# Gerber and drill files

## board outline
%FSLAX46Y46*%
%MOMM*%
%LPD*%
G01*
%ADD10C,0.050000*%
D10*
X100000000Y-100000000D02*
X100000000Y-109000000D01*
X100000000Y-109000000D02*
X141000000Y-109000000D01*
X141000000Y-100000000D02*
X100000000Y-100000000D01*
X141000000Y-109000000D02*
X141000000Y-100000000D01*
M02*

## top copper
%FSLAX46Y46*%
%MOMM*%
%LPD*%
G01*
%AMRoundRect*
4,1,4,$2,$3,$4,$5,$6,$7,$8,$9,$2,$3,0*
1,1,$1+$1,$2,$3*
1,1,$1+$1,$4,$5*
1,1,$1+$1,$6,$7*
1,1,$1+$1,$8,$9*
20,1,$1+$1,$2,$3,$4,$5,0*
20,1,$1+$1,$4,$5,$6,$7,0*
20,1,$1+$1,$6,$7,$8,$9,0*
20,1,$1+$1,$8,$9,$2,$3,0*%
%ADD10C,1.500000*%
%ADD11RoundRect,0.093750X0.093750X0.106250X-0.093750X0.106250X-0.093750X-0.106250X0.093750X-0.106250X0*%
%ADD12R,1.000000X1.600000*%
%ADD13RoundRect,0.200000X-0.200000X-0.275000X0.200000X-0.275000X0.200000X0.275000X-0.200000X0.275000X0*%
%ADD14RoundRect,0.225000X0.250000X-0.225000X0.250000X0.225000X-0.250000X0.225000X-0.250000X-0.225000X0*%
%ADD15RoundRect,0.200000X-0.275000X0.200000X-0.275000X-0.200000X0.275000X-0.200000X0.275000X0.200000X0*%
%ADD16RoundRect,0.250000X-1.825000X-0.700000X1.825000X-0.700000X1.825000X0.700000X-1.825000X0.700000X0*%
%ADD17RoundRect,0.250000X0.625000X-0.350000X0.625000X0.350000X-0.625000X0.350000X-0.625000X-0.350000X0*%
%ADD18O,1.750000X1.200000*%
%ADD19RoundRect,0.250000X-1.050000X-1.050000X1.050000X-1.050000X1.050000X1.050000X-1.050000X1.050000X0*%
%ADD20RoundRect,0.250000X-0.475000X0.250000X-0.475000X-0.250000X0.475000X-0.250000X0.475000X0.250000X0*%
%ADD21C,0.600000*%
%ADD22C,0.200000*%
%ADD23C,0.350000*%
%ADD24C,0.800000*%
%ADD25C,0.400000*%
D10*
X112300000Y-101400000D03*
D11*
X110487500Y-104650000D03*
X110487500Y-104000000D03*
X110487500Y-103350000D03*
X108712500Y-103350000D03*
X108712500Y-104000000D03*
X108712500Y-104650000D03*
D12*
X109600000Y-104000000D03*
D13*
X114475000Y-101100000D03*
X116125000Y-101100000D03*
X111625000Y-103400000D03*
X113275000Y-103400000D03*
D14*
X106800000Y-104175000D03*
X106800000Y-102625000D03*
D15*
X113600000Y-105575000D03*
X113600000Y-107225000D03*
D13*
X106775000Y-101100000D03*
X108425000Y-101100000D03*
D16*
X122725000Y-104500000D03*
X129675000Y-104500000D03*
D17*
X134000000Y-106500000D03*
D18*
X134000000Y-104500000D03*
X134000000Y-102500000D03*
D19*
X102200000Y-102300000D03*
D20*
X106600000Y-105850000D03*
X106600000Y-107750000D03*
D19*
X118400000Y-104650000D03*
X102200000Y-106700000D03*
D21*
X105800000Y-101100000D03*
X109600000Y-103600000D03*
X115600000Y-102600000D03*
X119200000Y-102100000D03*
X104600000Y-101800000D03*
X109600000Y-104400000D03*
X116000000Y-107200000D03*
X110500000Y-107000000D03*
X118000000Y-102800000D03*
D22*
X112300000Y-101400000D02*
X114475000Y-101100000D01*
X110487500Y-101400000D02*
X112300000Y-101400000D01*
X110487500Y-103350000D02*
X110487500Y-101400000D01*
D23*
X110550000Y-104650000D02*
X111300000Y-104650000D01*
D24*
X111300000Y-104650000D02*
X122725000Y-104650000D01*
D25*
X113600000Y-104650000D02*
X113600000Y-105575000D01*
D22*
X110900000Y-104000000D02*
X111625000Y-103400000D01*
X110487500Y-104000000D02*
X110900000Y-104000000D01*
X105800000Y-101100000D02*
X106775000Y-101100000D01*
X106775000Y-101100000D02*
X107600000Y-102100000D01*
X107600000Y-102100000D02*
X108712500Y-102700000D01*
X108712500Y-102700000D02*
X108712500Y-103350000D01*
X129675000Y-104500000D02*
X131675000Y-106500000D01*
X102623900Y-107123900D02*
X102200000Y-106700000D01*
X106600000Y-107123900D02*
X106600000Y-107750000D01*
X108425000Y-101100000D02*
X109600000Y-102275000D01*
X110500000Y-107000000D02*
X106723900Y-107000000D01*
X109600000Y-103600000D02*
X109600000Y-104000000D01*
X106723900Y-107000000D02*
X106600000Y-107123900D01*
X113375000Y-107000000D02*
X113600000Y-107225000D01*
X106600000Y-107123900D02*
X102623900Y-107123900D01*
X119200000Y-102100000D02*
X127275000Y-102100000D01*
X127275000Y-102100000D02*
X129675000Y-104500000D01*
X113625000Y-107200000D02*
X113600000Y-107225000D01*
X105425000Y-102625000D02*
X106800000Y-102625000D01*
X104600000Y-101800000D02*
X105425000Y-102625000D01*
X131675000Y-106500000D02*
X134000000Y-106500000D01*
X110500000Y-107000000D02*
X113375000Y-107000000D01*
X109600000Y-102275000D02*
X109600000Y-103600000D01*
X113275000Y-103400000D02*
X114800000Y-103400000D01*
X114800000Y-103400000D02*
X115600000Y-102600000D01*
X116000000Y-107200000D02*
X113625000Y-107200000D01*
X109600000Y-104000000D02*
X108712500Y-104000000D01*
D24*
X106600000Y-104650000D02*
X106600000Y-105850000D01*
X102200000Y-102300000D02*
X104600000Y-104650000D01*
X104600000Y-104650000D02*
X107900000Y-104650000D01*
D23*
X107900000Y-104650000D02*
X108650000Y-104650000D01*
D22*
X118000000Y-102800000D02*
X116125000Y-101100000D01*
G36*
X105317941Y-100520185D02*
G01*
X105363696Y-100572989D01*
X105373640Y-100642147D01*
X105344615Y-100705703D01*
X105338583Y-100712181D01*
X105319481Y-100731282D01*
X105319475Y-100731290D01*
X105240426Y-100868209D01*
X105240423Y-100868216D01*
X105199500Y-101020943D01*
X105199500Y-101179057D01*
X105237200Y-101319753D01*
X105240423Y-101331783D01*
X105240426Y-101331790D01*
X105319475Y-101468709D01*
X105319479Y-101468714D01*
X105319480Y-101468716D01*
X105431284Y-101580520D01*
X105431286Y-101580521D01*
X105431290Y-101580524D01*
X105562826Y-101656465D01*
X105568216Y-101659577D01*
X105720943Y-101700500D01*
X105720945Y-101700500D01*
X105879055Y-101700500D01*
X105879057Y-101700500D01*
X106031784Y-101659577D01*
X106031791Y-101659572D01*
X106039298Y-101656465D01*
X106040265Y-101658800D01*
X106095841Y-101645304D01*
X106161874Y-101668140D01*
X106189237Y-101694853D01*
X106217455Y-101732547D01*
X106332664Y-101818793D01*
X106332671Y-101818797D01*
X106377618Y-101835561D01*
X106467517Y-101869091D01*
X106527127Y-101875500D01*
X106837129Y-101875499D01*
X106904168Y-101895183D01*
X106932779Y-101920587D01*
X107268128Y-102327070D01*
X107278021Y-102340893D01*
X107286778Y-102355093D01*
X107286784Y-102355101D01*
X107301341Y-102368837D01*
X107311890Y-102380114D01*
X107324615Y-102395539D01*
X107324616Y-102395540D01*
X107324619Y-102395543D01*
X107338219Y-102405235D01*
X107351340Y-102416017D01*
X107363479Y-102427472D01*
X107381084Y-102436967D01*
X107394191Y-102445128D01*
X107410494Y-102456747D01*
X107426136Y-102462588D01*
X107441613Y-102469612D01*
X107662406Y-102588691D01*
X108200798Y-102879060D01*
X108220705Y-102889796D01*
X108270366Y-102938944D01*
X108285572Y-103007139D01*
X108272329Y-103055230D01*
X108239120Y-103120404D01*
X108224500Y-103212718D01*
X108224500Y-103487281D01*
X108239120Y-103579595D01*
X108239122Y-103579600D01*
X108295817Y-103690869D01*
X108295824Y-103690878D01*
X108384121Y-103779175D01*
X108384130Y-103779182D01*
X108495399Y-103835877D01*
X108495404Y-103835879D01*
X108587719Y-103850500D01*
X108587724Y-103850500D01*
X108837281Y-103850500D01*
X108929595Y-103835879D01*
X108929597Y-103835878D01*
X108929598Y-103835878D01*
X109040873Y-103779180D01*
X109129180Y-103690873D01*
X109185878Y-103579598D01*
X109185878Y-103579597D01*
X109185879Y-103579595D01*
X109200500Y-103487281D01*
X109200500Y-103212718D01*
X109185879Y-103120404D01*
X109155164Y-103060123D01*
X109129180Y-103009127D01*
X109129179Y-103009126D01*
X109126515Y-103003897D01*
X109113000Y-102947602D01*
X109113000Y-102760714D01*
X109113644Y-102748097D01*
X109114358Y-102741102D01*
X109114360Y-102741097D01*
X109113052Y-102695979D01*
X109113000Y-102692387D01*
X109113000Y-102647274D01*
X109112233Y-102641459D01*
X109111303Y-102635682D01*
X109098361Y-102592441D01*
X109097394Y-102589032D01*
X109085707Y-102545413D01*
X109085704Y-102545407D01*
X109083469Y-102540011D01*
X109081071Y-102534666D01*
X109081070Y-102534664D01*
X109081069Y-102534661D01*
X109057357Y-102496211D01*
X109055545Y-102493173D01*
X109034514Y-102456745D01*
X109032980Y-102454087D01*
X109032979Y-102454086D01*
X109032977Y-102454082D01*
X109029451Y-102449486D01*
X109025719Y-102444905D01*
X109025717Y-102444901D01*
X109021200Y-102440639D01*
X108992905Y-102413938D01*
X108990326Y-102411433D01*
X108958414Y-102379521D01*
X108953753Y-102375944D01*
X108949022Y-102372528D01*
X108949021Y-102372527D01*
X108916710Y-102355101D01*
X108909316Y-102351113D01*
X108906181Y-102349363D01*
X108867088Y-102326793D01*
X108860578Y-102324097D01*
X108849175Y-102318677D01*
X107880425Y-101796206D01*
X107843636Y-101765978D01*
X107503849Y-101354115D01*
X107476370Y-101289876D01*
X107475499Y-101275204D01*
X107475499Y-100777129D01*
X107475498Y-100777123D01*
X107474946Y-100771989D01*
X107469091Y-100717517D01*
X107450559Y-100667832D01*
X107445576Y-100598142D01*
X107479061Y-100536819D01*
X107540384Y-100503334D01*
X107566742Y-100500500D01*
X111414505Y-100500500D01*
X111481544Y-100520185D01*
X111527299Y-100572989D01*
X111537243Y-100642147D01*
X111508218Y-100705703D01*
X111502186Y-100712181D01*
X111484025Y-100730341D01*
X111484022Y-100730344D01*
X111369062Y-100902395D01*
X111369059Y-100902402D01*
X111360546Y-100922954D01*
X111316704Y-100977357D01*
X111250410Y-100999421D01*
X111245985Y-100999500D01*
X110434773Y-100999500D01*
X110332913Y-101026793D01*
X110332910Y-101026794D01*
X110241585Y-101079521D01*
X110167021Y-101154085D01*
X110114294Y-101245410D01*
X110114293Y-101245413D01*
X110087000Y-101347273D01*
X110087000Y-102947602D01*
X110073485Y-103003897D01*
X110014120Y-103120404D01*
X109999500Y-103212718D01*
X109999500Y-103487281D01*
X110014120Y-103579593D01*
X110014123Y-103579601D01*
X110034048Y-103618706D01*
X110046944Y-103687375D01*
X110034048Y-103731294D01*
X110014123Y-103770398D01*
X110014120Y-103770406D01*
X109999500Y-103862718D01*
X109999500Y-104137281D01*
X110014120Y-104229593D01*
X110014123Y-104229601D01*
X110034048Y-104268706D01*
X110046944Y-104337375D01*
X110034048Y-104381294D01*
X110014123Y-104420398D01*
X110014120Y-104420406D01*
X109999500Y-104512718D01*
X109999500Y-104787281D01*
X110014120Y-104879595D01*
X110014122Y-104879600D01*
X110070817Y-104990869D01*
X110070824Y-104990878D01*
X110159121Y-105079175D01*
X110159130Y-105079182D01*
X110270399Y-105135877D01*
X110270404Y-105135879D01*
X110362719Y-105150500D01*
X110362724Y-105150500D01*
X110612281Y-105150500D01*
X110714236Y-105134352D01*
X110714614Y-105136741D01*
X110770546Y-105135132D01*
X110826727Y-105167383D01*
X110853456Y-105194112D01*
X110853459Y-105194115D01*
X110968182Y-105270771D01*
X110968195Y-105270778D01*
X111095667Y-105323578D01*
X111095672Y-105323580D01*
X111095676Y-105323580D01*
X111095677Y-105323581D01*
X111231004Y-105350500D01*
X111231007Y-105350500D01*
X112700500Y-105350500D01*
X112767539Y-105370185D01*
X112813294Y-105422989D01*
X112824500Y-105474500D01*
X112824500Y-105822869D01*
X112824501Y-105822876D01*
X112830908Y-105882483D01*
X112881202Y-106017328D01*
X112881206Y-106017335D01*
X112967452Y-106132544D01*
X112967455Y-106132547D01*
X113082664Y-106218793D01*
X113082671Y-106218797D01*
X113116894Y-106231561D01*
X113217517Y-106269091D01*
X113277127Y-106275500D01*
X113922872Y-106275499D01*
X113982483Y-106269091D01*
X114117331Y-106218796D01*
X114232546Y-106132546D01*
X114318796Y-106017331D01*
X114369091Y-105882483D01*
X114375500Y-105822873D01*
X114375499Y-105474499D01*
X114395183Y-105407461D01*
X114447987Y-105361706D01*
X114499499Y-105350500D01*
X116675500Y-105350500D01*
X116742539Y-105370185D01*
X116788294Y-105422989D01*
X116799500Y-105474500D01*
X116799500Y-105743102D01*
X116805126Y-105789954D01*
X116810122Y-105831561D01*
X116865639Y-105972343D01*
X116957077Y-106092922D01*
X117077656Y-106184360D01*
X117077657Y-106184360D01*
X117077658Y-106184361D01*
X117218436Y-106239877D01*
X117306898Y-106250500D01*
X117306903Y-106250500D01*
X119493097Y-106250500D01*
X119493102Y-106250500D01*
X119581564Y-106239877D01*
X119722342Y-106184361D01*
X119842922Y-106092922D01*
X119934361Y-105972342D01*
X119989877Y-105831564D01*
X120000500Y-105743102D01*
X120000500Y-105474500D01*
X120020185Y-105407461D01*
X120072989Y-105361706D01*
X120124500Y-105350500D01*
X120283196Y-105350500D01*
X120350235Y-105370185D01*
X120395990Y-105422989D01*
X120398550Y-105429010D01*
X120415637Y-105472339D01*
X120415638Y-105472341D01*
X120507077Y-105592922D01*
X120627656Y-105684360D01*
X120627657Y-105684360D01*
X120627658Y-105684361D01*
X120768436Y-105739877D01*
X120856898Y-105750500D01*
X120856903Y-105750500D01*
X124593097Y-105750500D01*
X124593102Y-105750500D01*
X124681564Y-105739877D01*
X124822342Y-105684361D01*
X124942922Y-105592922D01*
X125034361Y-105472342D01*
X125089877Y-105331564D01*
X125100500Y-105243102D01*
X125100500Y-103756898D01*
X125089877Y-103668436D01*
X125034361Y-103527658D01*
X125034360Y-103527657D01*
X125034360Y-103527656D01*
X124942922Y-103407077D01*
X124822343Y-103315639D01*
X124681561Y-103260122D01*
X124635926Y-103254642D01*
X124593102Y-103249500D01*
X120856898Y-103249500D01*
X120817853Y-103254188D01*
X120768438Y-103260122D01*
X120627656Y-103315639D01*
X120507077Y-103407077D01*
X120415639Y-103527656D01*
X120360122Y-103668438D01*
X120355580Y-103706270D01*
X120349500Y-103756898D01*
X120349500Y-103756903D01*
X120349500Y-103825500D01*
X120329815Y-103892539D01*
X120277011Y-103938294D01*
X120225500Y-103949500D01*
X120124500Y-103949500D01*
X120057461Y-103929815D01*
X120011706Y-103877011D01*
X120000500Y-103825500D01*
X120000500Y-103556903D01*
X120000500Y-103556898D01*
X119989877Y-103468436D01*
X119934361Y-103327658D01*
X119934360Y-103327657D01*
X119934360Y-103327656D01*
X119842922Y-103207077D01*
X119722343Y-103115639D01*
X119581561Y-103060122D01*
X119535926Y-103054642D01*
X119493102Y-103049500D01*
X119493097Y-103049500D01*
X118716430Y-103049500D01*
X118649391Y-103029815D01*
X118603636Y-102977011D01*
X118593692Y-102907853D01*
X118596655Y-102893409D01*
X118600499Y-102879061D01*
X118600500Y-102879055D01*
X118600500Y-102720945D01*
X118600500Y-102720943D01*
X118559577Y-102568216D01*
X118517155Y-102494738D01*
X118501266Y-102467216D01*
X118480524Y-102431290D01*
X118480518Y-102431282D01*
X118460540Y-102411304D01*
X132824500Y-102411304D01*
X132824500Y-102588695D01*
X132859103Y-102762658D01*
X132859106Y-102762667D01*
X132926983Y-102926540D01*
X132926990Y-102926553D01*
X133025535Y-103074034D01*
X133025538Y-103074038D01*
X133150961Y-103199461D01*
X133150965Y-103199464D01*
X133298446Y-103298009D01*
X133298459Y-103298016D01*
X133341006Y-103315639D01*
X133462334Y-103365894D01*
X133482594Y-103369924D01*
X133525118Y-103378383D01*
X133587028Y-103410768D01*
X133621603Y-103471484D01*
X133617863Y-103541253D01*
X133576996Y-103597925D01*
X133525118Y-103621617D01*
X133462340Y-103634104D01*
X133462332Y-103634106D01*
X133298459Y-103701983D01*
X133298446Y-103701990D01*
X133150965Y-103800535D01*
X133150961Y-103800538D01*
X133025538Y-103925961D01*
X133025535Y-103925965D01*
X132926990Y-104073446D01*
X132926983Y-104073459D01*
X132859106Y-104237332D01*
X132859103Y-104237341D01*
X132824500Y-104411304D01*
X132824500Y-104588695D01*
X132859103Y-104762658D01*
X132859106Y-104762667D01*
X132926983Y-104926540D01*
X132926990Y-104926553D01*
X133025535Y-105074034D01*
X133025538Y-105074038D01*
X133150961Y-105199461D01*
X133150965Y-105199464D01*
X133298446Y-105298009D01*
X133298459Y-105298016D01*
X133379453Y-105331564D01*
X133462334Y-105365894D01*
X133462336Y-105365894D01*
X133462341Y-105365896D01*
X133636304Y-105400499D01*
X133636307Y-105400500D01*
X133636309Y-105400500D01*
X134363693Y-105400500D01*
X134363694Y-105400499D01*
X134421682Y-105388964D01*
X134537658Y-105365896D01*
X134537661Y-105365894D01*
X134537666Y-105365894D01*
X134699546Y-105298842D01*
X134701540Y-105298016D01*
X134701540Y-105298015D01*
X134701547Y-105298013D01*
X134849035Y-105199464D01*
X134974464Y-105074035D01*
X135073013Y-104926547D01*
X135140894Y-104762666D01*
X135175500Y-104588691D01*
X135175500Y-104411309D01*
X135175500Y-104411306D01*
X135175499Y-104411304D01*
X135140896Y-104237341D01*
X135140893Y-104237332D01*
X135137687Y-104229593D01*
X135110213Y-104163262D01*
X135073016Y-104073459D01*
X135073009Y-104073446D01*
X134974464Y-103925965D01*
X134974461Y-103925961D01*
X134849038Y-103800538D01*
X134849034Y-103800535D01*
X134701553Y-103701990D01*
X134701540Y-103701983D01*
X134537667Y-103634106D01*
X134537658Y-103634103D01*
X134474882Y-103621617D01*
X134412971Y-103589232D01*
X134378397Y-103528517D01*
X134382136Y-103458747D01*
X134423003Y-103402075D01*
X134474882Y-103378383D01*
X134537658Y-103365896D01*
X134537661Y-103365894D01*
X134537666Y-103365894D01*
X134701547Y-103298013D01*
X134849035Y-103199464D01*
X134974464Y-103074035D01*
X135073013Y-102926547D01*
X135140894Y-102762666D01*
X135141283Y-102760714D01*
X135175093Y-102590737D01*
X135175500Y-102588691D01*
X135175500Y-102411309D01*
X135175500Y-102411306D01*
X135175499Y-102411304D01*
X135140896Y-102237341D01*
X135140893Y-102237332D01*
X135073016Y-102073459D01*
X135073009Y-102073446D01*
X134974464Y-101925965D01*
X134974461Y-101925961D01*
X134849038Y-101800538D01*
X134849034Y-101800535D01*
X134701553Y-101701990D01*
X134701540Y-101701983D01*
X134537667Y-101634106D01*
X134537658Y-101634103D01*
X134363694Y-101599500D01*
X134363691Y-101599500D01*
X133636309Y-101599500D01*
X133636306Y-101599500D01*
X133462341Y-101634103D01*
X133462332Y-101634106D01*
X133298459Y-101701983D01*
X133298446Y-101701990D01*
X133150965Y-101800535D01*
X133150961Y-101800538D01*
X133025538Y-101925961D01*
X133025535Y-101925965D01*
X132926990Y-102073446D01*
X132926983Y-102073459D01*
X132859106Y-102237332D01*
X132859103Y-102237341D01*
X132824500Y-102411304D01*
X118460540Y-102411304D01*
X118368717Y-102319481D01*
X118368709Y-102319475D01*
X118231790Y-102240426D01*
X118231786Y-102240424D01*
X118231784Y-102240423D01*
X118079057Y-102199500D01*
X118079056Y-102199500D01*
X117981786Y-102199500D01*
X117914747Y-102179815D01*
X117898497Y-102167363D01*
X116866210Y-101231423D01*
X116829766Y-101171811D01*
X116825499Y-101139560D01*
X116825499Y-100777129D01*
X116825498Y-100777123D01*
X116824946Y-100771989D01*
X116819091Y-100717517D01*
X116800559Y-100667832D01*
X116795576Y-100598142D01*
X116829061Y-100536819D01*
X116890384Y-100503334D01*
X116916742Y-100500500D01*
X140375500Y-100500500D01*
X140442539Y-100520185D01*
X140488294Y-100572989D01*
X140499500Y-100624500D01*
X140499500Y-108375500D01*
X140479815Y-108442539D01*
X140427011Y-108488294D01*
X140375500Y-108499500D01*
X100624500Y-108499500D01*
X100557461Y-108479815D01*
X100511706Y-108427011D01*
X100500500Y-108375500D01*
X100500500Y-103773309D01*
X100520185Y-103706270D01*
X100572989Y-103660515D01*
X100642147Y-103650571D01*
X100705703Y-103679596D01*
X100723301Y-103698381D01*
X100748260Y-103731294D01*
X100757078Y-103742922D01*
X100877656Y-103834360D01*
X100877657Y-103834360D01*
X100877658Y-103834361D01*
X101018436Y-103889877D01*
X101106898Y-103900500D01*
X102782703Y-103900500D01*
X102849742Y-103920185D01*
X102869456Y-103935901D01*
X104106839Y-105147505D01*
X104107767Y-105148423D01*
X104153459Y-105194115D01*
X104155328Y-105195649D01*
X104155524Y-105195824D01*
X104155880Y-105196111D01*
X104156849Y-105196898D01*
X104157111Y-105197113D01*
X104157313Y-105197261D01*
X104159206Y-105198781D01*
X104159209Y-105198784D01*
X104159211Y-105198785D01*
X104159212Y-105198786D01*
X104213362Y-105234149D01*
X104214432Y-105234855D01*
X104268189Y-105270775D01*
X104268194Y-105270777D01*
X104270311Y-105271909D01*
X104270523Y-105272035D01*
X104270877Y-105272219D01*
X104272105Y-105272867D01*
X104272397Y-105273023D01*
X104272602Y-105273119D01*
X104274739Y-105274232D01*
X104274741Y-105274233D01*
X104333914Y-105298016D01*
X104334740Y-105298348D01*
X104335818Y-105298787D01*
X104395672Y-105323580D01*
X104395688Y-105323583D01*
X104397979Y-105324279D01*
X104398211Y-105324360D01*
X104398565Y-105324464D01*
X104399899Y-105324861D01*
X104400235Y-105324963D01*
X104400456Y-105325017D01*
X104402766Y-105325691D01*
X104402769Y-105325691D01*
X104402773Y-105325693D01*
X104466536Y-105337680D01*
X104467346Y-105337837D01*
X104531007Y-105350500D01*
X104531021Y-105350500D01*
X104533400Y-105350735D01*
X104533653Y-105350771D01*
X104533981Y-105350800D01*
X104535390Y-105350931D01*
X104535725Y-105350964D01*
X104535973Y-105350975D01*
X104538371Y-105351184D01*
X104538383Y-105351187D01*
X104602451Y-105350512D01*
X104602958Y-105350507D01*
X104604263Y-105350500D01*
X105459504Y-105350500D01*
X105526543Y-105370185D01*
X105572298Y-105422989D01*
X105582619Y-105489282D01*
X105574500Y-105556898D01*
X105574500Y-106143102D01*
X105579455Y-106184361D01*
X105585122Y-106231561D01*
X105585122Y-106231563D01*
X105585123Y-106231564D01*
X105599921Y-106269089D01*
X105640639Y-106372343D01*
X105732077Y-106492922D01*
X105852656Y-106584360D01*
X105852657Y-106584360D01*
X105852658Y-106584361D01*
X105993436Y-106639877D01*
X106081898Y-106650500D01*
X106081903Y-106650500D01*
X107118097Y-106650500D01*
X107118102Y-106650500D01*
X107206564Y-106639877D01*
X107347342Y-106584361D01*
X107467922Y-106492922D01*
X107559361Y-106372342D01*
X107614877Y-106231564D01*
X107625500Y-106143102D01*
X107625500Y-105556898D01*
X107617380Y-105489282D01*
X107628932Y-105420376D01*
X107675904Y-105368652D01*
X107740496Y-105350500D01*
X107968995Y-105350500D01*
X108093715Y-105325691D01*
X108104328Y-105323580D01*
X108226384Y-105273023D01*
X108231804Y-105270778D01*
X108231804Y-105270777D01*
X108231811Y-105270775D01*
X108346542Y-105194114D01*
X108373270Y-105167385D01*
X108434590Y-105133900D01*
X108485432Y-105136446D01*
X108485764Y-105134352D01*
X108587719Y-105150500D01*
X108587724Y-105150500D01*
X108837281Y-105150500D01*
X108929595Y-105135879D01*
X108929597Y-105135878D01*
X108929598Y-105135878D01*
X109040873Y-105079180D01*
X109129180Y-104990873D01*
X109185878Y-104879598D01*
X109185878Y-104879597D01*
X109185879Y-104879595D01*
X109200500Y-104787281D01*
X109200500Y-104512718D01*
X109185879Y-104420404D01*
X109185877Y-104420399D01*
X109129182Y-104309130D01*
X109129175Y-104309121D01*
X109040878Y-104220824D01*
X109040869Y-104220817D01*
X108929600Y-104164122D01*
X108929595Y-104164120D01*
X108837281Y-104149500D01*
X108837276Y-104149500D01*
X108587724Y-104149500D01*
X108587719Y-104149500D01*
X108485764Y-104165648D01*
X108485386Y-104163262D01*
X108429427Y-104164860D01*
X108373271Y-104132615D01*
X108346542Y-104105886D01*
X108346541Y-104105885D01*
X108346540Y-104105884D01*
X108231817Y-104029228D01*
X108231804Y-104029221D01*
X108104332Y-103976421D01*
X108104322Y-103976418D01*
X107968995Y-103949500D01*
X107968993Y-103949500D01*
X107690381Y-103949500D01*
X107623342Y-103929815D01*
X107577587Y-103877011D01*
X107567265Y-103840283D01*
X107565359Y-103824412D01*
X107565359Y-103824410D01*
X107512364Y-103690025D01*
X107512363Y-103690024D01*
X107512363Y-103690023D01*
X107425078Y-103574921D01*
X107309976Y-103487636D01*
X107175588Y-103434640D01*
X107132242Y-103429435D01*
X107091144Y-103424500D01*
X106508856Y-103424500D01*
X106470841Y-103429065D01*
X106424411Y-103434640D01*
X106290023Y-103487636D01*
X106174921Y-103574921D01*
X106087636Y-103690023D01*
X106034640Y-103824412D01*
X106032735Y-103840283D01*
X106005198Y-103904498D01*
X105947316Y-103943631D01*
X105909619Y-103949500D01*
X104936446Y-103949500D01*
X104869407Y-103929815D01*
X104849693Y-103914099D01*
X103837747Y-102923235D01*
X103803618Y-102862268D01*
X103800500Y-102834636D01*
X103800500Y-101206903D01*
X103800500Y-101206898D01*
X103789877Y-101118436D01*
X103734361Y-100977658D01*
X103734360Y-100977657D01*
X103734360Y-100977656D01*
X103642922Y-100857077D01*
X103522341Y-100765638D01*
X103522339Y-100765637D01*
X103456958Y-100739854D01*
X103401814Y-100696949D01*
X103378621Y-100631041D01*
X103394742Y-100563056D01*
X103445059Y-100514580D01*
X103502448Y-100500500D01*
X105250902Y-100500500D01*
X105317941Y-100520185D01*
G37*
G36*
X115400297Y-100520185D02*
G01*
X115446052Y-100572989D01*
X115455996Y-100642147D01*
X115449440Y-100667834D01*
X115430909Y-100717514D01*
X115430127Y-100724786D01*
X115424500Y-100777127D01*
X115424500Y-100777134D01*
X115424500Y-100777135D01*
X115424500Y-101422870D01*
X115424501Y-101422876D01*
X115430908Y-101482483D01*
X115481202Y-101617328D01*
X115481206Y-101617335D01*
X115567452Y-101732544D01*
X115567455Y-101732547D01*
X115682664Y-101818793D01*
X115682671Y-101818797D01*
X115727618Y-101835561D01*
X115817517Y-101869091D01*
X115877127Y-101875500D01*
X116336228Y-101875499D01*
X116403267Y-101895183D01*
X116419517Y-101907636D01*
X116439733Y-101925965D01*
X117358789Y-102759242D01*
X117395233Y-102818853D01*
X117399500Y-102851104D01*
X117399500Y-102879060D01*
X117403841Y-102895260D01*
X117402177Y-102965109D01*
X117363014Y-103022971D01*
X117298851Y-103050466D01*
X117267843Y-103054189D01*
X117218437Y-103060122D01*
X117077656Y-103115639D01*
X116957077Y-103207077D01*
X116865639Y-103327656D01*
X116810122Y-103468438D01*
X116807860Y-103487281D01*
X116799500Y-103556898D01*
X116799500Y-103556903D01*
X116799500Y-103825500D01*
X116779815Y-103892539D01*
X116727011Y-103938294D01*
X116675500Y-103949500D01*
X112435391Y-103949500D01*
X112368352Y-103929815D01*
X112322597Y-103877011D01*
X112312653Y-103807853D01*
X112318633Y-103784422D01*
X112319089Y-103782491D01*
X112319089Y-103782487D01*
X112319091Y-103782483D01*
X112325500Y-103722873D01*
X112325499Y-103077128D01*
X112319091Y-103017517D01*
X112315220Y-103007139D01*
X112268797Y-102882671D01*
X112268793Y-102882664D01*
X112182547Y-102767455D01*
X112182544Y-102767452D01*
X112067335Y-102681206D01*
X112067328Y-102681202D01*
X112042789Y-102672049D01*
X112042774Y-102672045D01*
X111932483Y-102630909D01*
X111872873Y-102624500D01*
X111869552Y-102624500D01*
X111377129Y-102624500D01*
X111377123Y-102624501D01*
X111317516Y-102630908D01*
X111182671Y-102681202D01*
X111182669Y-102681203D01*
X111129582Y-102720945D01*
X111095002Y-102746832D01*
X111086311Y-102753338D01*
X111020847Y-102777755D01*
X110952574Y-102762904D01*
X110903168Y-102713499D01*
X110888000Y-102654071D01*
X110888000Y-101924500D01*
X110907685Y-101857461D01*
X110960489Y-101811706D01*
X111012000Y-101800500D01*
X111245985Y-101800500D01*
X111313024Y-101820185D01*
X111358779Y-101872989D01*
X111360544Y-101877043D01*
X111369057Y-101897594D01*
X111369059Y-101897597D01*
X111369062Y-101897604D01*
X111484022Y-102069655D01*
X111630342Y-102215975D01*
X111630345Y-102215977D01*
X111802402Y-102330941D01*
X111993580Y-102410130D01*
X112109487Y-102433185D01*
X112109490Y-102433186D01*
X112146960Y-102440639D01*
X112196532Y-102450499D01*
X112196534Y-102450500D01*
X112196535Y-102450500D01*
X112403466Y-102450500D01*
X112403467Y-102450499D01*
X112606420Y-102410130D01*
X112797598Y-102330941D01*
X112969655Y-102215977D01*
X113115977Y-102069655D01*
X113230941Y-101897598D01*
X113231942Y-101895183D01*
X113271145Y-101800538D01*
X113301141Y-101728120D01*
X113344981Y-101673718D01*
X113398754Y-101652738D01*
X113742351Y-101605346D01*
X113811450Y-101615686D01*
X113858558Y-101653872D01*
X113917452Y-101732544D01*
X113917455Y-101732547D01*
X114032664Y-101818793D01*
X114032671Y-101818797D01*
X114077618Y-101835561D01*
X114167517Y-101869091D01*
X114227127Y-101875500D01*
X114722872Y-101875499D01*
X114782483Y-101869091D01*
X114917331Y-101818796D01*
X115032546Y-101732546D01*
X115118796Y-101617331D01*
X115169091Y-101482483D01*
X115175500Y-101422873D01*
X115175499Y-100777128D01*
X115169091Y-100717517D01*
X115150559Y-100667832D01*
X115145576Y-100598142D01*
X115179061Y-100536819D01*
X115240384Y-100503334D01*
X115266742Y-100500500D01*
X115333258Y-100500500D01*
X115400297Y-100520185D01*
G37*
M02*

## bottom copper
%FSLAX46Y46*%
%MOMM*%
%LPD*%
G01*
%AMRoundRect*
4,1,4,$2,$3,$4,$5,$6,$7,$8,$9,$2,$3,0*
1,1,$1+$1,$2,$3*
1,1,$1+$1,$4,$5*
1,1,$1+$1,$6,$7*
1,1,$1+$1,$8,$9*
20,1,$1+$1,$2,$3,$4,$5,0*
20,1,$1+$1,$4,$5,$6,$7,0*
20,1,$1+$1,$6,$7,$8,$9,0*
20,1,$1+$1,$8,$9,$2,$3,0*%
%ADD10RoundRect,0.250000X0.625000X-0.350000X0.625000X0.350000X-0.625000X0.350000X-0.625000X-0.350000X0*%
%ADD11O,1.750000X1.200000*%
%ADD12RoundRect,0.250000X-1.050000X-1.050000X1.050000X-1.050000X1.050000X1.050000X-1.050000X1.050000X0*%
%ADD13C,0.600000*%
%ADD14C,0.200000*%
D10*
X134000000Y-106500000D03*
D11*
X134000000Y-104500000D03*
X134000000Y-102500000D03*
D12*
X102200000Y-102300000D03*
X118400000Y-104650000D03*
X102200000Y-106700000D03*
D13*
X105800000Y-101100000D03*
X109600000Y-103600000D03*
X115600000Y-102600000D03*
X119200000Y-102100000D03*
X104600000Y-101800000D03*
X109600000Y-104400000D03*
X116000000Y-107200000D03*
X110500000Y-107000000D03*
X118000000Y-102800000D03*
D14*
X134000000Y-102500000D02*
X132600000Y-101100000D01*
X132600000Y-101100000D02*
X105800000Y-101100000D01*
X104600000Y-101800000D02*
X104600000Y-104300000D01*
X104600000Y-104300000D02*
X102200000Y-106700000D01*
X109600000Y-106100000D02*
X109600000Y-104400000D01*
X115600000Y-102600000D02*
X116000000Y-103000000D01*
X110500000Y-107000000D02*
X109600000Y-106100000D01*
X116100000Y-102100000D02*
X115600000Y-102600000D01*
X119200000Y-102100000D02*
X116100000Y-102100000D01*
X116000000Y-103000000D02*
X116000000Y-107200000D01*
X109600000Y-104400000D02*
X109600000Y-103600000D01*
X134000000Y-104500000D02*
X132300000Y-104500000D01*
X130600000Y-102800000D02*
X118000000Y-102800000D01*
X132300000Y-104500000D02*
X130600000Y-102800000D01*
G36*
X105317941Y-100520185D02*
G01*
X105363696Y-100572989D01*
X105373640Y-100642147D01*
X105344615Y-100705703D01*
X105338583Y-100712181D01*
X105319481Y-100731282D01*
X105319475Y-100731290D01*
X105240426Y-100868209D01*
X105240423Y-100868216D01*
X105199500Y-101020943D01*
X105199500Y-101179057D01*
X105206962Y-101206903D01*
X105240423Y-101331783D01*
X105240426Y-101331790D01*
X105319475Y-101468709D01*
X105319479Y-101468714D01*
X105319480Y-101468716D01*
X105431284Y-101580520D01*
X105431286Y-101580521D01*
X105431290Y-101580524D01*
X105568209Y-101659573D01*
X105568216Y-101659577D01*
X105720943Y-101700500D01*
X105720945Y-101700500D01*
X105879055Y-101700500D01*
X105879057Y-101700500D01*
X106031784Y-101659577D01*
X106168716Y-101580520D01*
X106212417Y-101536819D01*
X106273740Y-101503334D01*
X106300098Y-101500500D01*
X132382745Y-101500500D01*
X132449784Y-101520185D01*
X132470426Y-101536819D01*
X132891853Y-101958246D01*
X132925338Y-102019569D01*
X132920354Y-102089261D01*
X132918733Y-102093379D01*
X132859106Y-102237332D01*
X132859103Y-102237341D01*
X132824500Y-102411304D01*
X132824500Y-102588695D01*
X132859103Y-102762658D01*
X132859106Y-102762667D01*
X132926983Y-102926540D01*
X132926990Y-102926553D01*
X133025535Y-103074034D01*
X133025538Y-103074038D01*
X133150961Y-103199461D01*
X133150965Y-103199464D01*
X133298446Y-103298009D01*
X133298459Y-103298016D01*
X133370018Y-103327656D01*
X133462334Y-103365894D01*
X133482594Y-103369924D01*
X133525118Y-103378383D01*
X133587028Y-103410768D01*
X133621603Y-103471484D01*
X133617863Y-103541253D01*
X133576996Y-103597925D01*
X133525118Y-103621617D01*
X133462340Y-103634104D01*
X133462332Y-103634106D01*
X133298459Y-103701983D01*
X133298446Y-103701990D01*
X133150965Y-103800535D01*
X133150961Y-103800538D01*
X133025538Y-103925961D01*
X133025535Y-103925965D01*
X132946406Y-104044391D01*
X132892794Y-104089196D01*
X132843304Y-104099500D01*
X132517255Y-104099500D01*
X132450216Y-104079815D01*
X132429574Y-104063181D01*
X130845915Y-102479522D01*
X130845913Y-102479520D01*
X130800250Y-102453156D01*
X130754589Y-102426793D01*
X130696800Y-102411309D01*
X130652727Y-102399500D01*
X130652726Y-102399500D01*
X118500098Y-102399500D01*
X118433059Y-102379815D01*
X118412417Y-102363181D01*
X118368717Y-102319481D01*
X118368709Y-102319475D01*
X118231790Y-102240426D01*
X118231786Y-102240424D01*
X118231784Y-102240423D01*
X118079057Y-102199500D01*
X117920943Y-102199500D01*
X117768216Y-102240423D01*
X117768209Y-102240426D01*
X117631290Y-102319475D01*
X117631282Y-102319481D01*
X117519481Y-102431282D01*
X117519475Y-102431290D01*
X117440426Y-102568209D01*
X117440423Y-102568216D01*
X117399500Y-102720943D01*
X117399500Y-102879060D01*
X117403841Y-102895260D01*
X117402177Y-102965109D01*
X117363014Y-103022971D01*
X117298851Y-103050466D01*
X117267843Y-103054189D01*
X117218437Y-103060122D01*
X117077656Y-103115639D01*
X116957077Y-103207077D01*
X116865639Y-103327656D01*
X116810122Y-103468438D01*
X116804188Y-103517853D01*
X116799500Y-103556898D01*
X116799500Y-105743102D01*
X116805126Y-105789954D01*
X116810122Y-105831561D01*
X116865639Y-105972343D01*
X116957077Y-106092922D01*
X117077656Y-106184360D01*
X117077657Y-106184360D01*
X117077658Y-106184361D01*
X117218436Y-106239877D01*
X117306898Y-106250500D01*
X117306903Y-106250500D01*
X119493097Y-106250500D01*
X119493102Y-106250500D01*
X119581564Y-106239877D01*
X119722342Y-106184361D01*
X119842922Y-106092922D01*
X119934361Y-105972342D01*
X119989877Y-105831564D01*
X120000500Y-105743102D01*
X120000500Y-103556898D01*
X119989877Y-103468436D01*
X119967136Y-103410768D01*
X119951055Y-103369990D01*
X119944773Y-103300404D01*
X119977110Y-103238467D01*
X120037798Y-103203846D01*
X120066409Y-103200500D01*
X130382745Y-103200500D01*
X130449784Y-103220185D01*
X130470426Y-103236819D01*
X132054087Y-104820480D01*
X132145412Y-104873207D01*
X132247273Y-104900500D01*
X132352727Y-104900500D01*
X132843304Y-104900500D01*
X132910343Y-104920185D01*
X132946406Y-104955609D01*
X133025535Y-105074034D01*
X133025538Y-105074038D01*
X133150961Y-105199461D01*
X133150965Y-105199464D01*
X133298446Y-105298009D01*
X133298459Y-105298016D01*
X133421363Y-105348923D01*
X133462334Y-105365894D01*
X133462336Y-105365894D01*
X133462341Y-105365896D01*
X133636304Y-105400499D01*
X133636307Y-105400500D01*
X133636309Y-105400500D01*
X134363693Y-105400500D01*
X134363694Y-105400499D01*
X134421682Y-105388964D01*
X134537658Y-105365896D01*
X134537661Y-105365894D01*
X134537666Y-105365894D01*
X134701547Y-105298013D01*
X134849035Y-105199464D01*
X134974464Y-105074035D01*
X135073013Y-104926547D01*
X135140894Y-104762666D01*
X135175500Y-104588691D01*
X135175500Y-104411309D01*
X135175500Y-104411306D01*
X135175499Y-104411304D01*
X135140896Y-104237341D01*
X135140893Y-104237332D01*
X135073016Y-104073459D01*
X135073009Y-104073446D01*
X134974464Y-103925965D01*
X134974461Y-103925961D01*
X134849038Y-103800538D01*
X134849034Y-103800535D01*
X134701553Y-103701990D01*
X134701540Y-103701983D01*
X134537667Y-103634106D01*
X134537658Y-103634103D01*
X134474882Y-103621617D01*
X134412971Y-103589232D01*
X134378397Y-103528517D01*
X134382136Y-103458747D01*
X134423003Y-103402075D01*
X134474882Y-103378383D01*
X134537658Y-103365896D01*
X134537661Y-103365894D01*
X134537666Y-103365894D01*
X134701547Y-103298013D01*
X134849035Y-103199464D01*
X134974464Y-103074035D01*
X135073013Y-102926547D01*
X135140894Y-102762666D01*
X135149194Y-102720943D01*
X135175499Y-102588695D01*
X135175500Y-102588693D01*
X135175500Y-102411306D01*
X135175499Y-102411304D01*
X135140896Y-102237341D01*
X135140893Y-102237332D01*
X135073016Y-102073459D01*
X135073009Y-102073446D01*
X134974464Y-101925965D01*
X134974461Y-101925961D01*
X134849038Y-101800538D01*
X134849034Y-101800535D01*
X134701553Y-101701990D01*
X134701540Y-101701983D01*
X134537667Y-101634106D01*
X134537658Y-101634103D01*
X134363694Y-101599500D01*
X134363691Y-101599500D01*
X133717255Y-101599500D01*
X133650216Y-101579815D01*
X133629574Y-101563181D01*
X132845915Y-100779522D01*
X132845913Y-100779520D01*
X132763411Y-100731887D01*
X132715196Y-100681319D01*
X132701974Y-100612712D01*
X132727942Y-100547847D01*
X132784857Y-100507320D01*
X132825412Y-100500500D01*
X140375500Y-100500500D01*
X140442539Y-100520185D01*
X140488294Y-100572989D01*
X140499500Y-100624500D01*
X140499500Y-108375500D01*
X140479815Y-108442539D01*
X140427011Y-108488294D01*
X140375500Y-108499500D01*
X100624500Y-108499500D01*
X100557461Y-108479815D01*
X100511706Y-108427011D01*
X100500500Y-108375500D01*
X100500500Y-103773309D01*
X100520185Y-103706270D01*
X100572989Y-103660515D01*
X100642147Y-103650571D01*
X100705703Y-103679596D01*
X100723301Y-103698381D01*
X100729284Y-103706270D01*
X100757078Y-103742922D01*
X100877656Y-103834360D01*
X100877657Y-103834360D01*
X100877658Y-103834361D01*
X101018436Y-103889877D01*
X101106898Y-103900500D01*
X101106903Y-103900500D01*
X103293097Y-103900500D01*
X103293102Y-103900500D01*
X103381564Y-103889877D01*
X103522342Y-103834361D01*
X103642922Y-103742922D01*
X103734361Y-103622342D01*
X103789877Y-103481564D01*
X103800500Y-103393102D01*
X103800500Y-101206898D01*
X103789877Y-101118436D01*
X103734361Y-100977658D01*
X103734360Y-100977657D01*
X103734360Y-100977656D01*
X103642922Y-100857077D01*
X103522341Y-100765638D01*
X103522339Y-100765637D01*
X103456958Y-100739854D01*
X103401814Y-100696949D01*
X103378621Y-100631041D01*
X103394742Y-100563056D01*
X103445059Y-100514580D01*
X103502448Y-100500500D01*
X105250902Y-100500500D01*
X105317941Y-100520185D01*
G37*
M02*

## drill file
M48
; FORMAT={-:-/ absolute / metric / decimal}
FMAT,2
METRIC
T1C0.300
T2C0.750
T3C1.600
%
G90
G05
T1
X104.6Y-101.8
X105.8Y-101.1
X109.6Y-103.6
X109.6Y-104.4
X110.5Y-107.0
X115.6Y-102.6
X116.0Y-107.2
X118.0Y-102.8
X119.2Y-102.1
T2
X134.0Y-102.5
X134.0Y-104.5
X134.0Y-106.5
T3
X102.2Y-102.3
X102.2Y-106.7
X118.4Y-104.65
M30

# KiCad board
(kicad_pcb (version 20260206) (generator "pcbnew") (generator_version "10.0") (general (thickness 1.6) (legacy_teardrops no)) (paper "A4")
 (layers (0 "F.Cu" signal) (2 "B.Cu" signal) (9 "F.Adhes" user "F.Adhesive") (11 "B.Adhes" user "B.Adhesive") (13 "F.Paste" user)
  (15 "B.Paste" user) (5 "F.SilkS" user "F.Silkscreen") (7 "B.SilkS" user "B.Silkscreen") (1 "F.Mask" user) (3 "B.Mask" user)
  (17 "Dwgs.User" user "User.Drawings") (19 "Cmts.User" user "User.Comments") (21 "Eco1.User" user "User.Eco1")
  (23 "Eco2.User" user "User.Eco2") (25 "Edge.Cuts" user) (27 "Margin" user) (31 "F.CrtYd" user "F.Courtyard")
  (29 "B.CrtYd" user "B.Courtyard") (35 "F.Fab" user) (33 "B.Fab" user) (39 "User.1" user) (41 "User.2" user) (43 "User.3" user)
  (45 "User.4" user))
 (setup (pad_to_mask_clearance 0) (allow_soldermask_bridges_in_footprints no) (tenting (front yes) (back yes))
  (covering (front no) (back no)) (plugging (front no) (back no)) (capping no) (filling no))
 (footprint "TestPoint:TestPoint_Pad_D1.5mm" (layer "F.Cu") (at 112.3 101.4)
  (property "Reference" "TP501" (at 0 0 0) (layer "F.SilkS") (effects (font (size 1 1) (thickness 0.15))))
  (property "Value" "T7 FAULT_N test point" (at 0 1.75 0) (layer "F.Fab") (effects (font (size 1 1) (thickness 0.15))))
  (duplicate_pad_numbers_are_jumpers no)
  (pad "1" smd circle (at 0 0) (size 1.5 1.5) (layers "F.Cu" "F.Mask") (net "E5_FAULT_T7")))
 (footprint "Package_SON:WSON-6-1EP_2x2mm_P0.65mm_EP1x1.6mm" (layer "F.Cu") (at 109.6 104 180)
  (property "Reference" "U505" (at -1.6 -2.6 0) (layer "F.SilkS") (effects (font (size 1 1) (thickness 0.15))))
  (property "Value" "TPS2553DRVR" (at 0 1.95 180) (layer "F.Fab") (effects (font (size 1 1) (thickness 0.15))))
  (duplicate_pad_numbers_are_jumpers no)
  (pad "" smd roundrect (at 0 -0.4 180) (size 0.81 0.64) (layers "F.Paste") (roundrect_rratio 0.25))
  (pad "" smd roundrect (at 0 0.4 180) (size 0.81 0.64) (layers "F.Paste") (roundrect_rratio 0.25))
  (pad "1" smd roundrect (at -0.8875 -0.65 180) (size 0.375 0.4) (layers "F.Cu" "F.Mask" "F.Paste") (roundrect_rratio 0.25)
   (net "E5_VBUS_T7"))
  (pad "2" smd roundrect (at -0.8875 0 180) (size 0.375 0.4) (layers "F.Cu" "F.Mask" "F.Paste") (roundrect_rratio 0.25) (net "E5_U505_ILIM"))
  (pad "3" smd roundrect (at -0.8875 0.65 180) (size 0.375 0.4) (layers "F.Cu" "F.Mask" "F.Paste") (roundrect_rratio 0.25)
   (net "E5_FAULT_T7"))
  (pad "4" smd roundrect (at 0.8875 0.65 180) (size 0.375 0.4) (layers "F.Cu" "F.Mask" "F.Paste") (roundrect_rratio 0.25) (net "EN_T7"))
  (pad "5" smd roundrect (at 0.8875 0 180) (size 0.375 0.4) (layers "F.Cu" "F.Mask" "F.Paste") (roundrect_rratio 0.25) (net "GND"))
  (pad "6" smd roundrect (at 0.8875 -0.65 180) (size 0.375 0.4) (layers "F.Cu" "F.Mask" "F.Paste") (roundrect_rratio 0.25)
   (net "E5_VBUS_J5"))
  (pad "7" smd rect (at 0 0 180) (size 1 1.6) (layers "F.Cu" "F.Mask") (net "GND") (zone_connect 2)))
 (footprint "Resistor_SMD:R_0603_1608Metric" (layer "F.Cu") (at 115.3 101.1)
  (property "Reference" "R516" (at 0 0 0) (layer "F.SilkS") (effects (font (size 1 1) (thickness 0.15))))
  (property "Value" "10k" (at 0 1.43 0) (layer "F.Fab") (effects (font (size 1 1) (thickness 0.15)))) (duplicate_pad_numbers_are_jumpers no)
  (pad "1" smd roundrect (at -0.825 0) (size 0.8 0.95) (layers "F.Cu" "F.Mask" "F.Paste") (roundrect_rratio 0.25) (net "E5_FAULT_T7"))
  (pad "2" smd roundrect (at 0.825 0) (size 0.8 0.95) (layers "F.Cu" "F.Mask" "F.Paste") (roundrect_rratio 0.25) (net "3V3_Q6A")))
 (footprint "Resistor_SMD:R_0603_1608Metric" (layer "F.Cu") (at 112.45 103.4)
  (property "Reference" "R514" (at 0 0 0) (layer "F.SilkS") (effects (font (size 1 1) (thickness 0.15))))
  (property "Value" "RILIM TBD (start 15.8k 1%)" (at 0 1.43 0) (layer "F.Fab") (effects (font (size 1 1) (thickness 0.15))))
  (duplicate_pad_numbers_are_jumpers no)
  (pad "1" smd roundrect (at -0.825 0) (size 0.8 0.95) (layers "F.Cu" "F.Mask" "F.Paste") (roundrect_rratio 0.25) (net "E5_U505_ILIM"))
  (pad "2" smd roundrect (at 0.825 0) (size 0.8 0.95) (layers "F.Cu" "F.Mask" "F.Paste") (roundrect_rratio 0.25) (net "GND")))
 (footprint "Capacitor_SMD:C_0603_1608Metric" (layer "F.Cu") (at 106.8 103.4 90)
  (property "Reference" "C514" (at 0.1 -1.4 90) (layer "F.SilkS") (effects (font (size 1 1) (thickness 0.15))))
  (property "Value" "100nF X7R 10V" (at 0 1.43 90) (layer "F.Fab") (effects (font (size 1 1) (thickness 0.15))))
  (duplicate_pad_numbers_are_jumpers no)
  (pad "1" smd roundrect (at -0.775 0 90) (size 0.9 0.95) (layers "F.Cu" "F.Mask" "F.Paste") (roundrect_rratio 0.25) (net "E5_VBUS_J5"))
  (pad "2" smd roundrect (at 0.775 0 90) (size 0.9 0.95) (layers "F.Cu" "F.Mask" "F.Paste") (roundrect_rratio 0.25) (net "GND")))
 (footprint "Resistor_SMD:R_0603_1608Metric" (layer "F.Cu") (at 113.6 106.4 -90)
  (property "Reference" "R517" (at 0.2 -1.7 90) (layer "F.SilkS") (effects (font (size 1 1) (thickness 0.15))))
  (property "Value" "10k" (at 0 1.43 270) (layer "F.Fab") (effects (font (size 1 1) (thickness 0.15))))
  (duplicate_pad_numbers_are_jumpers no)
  (pad "1" smd roundrect (at -0.825 0 270) (size 0.8 0.95) (layers "F.Cu" "F.Mask" "F.Paste") (roundrect_rratio 0.25) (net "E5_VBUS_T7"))
  (pad "2" smd roundrect (at 0.825 0 270) (size 0.8 0.95) (layers "F.Cu" "F.Mask" "F.Paste") (roundrect_rratio 0.25) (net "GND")))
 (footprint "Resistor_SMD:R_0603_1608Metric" (layer "F.Cu") (at 107.6 101.1)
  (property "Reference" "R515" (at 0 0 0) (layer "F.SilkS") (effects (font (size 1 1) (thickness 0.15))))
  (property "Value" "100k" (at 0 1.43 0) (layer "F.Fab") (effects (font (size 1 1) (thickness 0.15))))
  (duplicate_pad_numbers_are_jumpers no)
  (pad "1" smd roundrect (at -0.825 0) (size 0.8 0.95) (layers "F.Cu" "F.Mask" "F.Paste") (roundrect_rratio 0.25) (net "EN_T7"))
  (pad "2" smd roundrect (at 0.825 0) (size 0.8 0.95) (layers "F.Cu" "F.Mask" "F.Paste") (roundrect_rratio 0.25) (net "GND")))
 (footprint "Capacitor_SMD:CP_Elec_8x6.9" (layer "F.Cu") (at 126.2 104.5)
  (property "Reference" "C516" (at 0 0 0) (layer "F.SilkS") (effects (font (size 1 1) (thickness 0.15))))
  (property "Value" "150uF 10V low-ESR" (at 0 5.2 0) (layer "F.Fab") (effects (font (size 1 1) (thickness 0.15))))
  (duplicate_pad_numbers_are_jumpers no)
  (pad "1" smd roundrect (at -3.475 0) (size 4.15 1.9) (layers "F.Cu" "F.Mask" "F.Paste") (roundrect_rratio 0.131579) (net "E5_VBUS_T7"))
  (pad "2" smd roundrect (at 3.475 0) (size 4.15 1.9) (layers "F.Cu" "F.Mask" "F.Paste") (roundrect_rratio 0.131579) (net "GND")))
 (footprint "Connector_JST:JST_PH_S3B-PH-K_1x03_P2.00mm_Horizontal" (layer "F.Cu") (at 134 106.5 90)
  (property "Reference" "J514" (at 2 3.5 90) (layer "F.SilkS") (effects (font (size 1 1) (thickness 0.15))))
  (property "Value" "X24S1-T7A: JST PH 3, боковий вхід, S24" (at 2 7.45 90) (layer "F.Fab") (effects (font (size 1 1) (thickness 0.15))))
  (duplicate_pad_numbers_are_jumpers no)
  (pad "1" thru_hole roundrect (at 0 0 90) (size 1.2 1.75) (drill 0.75) (layers "*.Cu" "*.Mask") (remove_unused_layers no)
   (roundrect_rratio 0.208333) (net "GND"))
  (pad "2" thru_hole oval (at 2 0 90) (size 1.2 1.75) (drill 0.75) (layers "*.Cu" "*.Mask") (remove_unused_layers no) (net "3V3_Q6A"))
  (pad "3" thru_hole oval (at 4 0 90) (size 1.2 1.75) (drill 0.75) (layers "*.Cu" "*.Mask") (remove_unused_layers no) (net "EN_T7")))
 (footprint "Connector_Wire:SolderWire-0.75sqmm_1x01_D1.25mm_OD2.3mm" (layer "F.Cu") (at 102.2 102.3)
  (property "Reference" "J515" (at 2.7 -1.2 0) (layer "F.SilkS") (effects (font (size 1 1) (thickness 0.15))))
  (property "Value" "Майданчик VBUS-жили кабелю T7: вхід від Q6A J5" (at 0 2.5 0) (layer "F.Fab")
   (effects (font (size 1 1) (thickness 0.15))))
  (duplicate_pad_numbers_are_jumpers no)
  (pad "1" thru_hole roundrect (at 0 0) (size 2.6 2.6) (drill 1.6) (layers "*.Cu" "*.Mask") (remove_unused_layers no)
   (roundrect_rratio 0.096154) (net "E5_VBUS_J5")))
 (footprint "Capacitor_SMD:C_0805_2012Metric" (layer "F.Cu") (at 106.6 106.8 -90)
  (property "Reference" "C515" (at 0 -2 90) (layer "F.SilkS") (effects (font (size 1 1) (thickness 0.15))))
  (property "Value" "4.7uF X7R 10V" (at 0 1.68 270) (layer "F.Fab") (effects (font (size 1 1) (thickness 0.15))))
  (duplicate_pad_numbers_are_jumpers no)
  (pad "1" smd roundrect (at -0.95 0 270) (size 1 1.45) (layers "F.Cu" "F.Mask" "F.Paste") (roundrect_rratio 0.25) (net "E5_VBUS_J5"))
  (pad "2" smd roundrect (at 0.95 0 270) (size 1 1.45) (layers "F.Cu" "F.Mask" "F.Paste") (roundrect_rratio 0.25) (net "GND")))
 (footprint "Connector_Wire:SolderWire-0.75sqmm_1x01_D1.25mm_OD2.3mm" (layer "F.Cu") (at 118.4 104.65)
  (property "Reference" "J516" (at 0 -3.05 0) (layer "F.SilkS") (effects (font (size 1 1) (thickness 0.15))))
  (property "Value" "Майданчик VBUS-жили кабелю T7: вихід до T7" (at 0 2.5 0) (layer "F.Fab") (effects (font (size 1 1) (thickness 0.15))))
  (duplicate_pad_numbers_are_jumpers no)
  (pad "1" thru_hole roundrect (at 0 0) (size 2.6 2.6) (drill 1.6) (layers "*.Cu" "*.Mask") (remove_unused_layers no)
   (roundrect_rratio 0.096154) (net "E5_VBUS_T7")))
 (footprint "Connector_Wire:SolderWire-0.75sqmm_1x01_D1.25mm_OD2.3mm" (layer "F.Cu") (at 102.2 106.7)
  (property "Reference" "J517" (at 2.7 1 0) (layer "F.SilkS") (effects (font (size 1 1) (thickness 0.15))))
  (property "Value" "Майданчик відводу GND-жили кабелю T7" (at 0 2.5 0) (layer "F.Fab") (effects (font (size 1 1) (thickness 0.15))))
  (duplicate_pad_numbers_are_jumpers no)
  (pad "1" thru_hole roundrect (at 0 0) (size 2.6 2.6) (drill 1.6) (layers "*.Cu" "*.Mask") (remove_unused_layers no)
   (roundrect_rratio 0.096154) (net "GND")))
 (gr_line (start 100 100) (end 100 109) (stroke (width 0.05) (type default)) (layer "Edge.Cuts"))
 (gr_line (start 100 109) (end 141 109) (stroke (width 0.05) (type default)) (layer "Edge.Cuts"))
 (gr_line (start 141 100) (end 100 100) (stroke (width 0.05) (type default)) (layer "Edge.Cuts"))
 (gr_line (start 141 109) (end 141 100) (stroke (width 0.05) (type default)) (layer "Edge.Cuts"))
 (segment (start 112.3 101.4) (end 114.475 101.1) (width 0.2) (locked yes) (layer "F.Cu") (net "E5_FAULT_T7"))
 (segment (start 110.4875 101.4) (end 112.3 101.4) (width 0.2) (locked yes) (layer "F.Cu") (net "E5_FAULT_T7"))
 (segment (start 110.4875 103.35) (end 110.4875 101.4) (width 0.2) (locked yes) (layer "F.Cu") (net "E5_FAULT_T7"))
 (segment (start 110.55 104.65) (end 111.3 104.65) (width 0.35) (locked yes) (layer "F.Cu") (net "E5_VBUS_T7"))
 (segment (start 111.3 104.65) (end 122.725 104.65) (width 0.8) (locked yes) (layer "F.Cu") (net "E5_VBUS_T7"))
 (segment (start 113.6 104.65) (end 113.6 105.575) (width 0.4) (locked yes) (layer "F.Cu") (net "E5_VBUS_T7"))
 (segment (start 110.9 104) (end 111.625 103.4) (width 0.2) (locked yes) (layer "F.Cu") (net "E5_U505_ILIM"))
 (segment (start 110.4875 104) (end 110.9 104) (width 0.2) (locked yes) (layer "F.Cu") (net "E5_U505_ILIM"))
 (segment (start 105.8 101.1) (end 106.775 101.1) (width 0.2) (locked yes) (layer "F.Cu") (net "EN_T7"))
 (segment (start 106.775 101.1) (end 107.6 102.1) (width 0.2) (locked yes) (layer "F.Cu") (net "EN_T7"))
 (segment (start 107.6 102.1) (end 108.7125 102.7) (width 0.2) (locked yes) (layer "F.Cu") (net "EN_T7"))
 (segment (start 108.7125 102.7) (end 108.7125 103.35) (width 0.2) (locked yes) (layer "F.Cu") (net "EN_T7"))
 (via (at 105.8 101.1) (size 0.6) (drill 0.3) (layers "F.Cu" "B.Cu") (locked yes) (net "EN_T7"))
 (segment (start 134 102.5) (end 132.6 101.1) (width 0.2) (locked yes) (layer "B.Cu") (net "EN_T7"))
 (segment (start 132.6 101.1) (end 105.8 101.1) (width 0.2) (locked yes) (layer "B.Cu") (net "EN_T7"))
 (segment (start 129.675 104.5) (end 131.675 106.5) (width 0.2) (layer "F.Cu") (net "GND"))
 (segment (start 102.6239 107.1239) (end 102.2 106.7) (width 0.2) (layer "F.Cu") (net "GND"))
 (segment (start 106.6 107.1239) (end 106.6 107.75) (width 0.2) (layer "F.Cu") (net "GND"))
 (segment (start 108.425 101.1) (end 109.6 102.275) (width 0.2) (layer "F.Cu") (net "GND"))
 (segment (start 110.5 107) (end 106.7239 107) (width 0.2) (layer "F.Cu") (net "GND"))
 (segment (start 109.6 103.6) (end 109.6 104) (width 0.2) (layer "F.Cu") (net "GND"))
 (segment (start 106.7239 107) (end 106.6 107.1239) (width 0.2) (layer "F.Cu") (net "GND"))
 (segment (start 113.375 107) (end 113.6 107.225) (width 0.2) (layer "F.Cu") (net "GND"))
 (segment (start 106.6 107.1239) (end 102.6239 107.1239) (width 0.2) (layer "F.Cu") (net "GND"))
 (segment (start 119.2 102.1) (end 127.275 102.1) (width 0.2) (layer "F.Cu") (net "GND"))
 (segment (start 127.275 102.1) (end 129.675 104.5) (width 0.2) (layer "F.Cu") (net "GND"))
 (segment (start 113.625 107.2) (end 113.6 107.225) (width 0.2) (layer "F.Cu") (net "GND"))
 (segment (start 105.425 102.625) (end 106.8 102.625) (width 0.2) (layer "F.Cu") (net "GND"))
 (segment (start 104.6 101.8) (end 105.425 102.625) (width 0.2) (layer "F.Cu") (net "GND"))
 (segment (start 131.675 106.5) (end 134 106.5) (width 0.2) (layer "F.Cu") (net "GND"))
 (segment (start 110.5 107) (end 113.375 107) (width 0.2) (layer "F.Cu") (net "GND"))
 (segment (start 109.6 102.275) (end 109.6 103.6) (width 0.2) (layer "F.Cu") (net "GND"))
 (segment (start 113.275 103.4) (end 114.8 103.4) (width 0.2) (layer "F.Cu") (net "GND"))
 (segment (start 114.8 103.4) (end 115.6 102.6) (width 0.2) (layer "F.Cu") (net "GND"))
 (segment (start 116 107.2) (end 113.625 107.2) (width 0.2) (layer "F.Cu") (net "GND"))
 (segment (start 109.6 104) (end 108.7125 104) (width 0.2) (layer "F.Cu") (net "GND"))
 (via (at 109.6 103.6) (size 0.6) (drill 0.3) (layers "F.Cu" "B.Cu") (locked yes) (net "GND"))
 (via (at 115.6 102.6) (size 0.6) (drill 0.3) (layers "F.Cu" "B.Cu") (locked yes) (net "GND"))
 (via (at 119.2 102.1) (size 0.6) (drill 0.3) (layers "F.Cu" "B.Cu") (locked yes) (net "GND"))
 (via (at 104.6 101.8) (size 0.6) (drill 0.3) (layers "F.Cu" "B.Cu") (locked yes) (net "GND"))
 (via (at 109.6 104.4) (size 0.6) (drill 0.3) (layers "F.Cu" "B.Cu") (locked yes) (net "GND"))
 (via (at 116 107.2) (size 0.6) (drill 0.3) (layers "F.Cu" "B.Cu") (locked yes) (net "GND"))
 (via (at 110.5 107) (size 0.6) (drill 0.3) (layers "F.Cu" "B.Cu") (locked yes) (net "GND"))
 (segment (start 104.6 101.8) (end 104.6 104.3) (width 0.2) (layer "B.Cu") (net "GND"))
 (segment (start 104.6 104.3) (end 102.2 106.7) (width 0.2) (layer "B.Cu") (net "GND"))
 (segment (start 109.6 106.1) (end 109.6 104.4) (width 0.2) (layer "B.Cu") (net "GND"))
 (segment (start 115.6 102.6) (end 116 103) (width 0.2) (layer "B.Cu") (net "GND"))
 (segment (start 110.5 107) (end 109.6 106.1) (width 0.2) (layer "B.Cu") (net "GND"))
 (segment (start 116.1 102.1) (end 115.6 102.6) (width 0.2) (layer "B.Cu") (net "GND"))
 (segment (start 119.2 102.1) (end 116.1 102.1) (width 0.2) (layer "B.Cu") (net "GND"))
 (segment (start 116 103) (end 116 107.2) (width 0.2) (layer "B.Cu") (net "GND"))
 (segment (start 109.6 104.4) (end 109.6 103.6) (width 0.2) (layer "B.Cu") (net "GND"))
 (segment (start 106.6 104.65) (end 106.6 105.85) (width 0.8) (locked yes) (layer "F.Cu") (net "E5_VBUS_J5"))
 (segment (start 102.2 102.3) (end 104.6 104.65) (width 0.8) (locked yes) (layer "F.Cu") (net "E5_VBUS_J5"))
 (segment (start 104.6 104.65) (end 107.9 104.65) (width 0.8) (locked yes) (layer "F.Cu") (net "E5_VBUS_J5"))
 (segment (start 107.9 104.65) (end 108.65 104.65) (width 0.35) (locked yes) (layer "F.Cu") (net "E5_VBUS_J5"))
 (segment (start 118 102.8) (end 116.125 101.1) (width 0.2) (locked yes) (layer "F.Cu") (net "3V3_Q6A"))
 (via (at 118 102.8) (size 0.6) (drill 0.3) (layers "F.Cu" "B.Cu") (locked yes) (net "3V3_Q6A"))
 (segment (start 134 104.5) (end 132.3 104.5) (width 0.2) (locked yes) (layer "B.Cu") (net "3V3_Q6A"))
 (segment (start 130.6 102.8) (end 118 102.8) (width 0.2) (locked yes) (layer "B.Cu") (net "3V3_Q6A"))
 (segment (start 132.3 104.5) (end 130.6 102.8) (width 0.2) (locked yes) (layer "B.Cu") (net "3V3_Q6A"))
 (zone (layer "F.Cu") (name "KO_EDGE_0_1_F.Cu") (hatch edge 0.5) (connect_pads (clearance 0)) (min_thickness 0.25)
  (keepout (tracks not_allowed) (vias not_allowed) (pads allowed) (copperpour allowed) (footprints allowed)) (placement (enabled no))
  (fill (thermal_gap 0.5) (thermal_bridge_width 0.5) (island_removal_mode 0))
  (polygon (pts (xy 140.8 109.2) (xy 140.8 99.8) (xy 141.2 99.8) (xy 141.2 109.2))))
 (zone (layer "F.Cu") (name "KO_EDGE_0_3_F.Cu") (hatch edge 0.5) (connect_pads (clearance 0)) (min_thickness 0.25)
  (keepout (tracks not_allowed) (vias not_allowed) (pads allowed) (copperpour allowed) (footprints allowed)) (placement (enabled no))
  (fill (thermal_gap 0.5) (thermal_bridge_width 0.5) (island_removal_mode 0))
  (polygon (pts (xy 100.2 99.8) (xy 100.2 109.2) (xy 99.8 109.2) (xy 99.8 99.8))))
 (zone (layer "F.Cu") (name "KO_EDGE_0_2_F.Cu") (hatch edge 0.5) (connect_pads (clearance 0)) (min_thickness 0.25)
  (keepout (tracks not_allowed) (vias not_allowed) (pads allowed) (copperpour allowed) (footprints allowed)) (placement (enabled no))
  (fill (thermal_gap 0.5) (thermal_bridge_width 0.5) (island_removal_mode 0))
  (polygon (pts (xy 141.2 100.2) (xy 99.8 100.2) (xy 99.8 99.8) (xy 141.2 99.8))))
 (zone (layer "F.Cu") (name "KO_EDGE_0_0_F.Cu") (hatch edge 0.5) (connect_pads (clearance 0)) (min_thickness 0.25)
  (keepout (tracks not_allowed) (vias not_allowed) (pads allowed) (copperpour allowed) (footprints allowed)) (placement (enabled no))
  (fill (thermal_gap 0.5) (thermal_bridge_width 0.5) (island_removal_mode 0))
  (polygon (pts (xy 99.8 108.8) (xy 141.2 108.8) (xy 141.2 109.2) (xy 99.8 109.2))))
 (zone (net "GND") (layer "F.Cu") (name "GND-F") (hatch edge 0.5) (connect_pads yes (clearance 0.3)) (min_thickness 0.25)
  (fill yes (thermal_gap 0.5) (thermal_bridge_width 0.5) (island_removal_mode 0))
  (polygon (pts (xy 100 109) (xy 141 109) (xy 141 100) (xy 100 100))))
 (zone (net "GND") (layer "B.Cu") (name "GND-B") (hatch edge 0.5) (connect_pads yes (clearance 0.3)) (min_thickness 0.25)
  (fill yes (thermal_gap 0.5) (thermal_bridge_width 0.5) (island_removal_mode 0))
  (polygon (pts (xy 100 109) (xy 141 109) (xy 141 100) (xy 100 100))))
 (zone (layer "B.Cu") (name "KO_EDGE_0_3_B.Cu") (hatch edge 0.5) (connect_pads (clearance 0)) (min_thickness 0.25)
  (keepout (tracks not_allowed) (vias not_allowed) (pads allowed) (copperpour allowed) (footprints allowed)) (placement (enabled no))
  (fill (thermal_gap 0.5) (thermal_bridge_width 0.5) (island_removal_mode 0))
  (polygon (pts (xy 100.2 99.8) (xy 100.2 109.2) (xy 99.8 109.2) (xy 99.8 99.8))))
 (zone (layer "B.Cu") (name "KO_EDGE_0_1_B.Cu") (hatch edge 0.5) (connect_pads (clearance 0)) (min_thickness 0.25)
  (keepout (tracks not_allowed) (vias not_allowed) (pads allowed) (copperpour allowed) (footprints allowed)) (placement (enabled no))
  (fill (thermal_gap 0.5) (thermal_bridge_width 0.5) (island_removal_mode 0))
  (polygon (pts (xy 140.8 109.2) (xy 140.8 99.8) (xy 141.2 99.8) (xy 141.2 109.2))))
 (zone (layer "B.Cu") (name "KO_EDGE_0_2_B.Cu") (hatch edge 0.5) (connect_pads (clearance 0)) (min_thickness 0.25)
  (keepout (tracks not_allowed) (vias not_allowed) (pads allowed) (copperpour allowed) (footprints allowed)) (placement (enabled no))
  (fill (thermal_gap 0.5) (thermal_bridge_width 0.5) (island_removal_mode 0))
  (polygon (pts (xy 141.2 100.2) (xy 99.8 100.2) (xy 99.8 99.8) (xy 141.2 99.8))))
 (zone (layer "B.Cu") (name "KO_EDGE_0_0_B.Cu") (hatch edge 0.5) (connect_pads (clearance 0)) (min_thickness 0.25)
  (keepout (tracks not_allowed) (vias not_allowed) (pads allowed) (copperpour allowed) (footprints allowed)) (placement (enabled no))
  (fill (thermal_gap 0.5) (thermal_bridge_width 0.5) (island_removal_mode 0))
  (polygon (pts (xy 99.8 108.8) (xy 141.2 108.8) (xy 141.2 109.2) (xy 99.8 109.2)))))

